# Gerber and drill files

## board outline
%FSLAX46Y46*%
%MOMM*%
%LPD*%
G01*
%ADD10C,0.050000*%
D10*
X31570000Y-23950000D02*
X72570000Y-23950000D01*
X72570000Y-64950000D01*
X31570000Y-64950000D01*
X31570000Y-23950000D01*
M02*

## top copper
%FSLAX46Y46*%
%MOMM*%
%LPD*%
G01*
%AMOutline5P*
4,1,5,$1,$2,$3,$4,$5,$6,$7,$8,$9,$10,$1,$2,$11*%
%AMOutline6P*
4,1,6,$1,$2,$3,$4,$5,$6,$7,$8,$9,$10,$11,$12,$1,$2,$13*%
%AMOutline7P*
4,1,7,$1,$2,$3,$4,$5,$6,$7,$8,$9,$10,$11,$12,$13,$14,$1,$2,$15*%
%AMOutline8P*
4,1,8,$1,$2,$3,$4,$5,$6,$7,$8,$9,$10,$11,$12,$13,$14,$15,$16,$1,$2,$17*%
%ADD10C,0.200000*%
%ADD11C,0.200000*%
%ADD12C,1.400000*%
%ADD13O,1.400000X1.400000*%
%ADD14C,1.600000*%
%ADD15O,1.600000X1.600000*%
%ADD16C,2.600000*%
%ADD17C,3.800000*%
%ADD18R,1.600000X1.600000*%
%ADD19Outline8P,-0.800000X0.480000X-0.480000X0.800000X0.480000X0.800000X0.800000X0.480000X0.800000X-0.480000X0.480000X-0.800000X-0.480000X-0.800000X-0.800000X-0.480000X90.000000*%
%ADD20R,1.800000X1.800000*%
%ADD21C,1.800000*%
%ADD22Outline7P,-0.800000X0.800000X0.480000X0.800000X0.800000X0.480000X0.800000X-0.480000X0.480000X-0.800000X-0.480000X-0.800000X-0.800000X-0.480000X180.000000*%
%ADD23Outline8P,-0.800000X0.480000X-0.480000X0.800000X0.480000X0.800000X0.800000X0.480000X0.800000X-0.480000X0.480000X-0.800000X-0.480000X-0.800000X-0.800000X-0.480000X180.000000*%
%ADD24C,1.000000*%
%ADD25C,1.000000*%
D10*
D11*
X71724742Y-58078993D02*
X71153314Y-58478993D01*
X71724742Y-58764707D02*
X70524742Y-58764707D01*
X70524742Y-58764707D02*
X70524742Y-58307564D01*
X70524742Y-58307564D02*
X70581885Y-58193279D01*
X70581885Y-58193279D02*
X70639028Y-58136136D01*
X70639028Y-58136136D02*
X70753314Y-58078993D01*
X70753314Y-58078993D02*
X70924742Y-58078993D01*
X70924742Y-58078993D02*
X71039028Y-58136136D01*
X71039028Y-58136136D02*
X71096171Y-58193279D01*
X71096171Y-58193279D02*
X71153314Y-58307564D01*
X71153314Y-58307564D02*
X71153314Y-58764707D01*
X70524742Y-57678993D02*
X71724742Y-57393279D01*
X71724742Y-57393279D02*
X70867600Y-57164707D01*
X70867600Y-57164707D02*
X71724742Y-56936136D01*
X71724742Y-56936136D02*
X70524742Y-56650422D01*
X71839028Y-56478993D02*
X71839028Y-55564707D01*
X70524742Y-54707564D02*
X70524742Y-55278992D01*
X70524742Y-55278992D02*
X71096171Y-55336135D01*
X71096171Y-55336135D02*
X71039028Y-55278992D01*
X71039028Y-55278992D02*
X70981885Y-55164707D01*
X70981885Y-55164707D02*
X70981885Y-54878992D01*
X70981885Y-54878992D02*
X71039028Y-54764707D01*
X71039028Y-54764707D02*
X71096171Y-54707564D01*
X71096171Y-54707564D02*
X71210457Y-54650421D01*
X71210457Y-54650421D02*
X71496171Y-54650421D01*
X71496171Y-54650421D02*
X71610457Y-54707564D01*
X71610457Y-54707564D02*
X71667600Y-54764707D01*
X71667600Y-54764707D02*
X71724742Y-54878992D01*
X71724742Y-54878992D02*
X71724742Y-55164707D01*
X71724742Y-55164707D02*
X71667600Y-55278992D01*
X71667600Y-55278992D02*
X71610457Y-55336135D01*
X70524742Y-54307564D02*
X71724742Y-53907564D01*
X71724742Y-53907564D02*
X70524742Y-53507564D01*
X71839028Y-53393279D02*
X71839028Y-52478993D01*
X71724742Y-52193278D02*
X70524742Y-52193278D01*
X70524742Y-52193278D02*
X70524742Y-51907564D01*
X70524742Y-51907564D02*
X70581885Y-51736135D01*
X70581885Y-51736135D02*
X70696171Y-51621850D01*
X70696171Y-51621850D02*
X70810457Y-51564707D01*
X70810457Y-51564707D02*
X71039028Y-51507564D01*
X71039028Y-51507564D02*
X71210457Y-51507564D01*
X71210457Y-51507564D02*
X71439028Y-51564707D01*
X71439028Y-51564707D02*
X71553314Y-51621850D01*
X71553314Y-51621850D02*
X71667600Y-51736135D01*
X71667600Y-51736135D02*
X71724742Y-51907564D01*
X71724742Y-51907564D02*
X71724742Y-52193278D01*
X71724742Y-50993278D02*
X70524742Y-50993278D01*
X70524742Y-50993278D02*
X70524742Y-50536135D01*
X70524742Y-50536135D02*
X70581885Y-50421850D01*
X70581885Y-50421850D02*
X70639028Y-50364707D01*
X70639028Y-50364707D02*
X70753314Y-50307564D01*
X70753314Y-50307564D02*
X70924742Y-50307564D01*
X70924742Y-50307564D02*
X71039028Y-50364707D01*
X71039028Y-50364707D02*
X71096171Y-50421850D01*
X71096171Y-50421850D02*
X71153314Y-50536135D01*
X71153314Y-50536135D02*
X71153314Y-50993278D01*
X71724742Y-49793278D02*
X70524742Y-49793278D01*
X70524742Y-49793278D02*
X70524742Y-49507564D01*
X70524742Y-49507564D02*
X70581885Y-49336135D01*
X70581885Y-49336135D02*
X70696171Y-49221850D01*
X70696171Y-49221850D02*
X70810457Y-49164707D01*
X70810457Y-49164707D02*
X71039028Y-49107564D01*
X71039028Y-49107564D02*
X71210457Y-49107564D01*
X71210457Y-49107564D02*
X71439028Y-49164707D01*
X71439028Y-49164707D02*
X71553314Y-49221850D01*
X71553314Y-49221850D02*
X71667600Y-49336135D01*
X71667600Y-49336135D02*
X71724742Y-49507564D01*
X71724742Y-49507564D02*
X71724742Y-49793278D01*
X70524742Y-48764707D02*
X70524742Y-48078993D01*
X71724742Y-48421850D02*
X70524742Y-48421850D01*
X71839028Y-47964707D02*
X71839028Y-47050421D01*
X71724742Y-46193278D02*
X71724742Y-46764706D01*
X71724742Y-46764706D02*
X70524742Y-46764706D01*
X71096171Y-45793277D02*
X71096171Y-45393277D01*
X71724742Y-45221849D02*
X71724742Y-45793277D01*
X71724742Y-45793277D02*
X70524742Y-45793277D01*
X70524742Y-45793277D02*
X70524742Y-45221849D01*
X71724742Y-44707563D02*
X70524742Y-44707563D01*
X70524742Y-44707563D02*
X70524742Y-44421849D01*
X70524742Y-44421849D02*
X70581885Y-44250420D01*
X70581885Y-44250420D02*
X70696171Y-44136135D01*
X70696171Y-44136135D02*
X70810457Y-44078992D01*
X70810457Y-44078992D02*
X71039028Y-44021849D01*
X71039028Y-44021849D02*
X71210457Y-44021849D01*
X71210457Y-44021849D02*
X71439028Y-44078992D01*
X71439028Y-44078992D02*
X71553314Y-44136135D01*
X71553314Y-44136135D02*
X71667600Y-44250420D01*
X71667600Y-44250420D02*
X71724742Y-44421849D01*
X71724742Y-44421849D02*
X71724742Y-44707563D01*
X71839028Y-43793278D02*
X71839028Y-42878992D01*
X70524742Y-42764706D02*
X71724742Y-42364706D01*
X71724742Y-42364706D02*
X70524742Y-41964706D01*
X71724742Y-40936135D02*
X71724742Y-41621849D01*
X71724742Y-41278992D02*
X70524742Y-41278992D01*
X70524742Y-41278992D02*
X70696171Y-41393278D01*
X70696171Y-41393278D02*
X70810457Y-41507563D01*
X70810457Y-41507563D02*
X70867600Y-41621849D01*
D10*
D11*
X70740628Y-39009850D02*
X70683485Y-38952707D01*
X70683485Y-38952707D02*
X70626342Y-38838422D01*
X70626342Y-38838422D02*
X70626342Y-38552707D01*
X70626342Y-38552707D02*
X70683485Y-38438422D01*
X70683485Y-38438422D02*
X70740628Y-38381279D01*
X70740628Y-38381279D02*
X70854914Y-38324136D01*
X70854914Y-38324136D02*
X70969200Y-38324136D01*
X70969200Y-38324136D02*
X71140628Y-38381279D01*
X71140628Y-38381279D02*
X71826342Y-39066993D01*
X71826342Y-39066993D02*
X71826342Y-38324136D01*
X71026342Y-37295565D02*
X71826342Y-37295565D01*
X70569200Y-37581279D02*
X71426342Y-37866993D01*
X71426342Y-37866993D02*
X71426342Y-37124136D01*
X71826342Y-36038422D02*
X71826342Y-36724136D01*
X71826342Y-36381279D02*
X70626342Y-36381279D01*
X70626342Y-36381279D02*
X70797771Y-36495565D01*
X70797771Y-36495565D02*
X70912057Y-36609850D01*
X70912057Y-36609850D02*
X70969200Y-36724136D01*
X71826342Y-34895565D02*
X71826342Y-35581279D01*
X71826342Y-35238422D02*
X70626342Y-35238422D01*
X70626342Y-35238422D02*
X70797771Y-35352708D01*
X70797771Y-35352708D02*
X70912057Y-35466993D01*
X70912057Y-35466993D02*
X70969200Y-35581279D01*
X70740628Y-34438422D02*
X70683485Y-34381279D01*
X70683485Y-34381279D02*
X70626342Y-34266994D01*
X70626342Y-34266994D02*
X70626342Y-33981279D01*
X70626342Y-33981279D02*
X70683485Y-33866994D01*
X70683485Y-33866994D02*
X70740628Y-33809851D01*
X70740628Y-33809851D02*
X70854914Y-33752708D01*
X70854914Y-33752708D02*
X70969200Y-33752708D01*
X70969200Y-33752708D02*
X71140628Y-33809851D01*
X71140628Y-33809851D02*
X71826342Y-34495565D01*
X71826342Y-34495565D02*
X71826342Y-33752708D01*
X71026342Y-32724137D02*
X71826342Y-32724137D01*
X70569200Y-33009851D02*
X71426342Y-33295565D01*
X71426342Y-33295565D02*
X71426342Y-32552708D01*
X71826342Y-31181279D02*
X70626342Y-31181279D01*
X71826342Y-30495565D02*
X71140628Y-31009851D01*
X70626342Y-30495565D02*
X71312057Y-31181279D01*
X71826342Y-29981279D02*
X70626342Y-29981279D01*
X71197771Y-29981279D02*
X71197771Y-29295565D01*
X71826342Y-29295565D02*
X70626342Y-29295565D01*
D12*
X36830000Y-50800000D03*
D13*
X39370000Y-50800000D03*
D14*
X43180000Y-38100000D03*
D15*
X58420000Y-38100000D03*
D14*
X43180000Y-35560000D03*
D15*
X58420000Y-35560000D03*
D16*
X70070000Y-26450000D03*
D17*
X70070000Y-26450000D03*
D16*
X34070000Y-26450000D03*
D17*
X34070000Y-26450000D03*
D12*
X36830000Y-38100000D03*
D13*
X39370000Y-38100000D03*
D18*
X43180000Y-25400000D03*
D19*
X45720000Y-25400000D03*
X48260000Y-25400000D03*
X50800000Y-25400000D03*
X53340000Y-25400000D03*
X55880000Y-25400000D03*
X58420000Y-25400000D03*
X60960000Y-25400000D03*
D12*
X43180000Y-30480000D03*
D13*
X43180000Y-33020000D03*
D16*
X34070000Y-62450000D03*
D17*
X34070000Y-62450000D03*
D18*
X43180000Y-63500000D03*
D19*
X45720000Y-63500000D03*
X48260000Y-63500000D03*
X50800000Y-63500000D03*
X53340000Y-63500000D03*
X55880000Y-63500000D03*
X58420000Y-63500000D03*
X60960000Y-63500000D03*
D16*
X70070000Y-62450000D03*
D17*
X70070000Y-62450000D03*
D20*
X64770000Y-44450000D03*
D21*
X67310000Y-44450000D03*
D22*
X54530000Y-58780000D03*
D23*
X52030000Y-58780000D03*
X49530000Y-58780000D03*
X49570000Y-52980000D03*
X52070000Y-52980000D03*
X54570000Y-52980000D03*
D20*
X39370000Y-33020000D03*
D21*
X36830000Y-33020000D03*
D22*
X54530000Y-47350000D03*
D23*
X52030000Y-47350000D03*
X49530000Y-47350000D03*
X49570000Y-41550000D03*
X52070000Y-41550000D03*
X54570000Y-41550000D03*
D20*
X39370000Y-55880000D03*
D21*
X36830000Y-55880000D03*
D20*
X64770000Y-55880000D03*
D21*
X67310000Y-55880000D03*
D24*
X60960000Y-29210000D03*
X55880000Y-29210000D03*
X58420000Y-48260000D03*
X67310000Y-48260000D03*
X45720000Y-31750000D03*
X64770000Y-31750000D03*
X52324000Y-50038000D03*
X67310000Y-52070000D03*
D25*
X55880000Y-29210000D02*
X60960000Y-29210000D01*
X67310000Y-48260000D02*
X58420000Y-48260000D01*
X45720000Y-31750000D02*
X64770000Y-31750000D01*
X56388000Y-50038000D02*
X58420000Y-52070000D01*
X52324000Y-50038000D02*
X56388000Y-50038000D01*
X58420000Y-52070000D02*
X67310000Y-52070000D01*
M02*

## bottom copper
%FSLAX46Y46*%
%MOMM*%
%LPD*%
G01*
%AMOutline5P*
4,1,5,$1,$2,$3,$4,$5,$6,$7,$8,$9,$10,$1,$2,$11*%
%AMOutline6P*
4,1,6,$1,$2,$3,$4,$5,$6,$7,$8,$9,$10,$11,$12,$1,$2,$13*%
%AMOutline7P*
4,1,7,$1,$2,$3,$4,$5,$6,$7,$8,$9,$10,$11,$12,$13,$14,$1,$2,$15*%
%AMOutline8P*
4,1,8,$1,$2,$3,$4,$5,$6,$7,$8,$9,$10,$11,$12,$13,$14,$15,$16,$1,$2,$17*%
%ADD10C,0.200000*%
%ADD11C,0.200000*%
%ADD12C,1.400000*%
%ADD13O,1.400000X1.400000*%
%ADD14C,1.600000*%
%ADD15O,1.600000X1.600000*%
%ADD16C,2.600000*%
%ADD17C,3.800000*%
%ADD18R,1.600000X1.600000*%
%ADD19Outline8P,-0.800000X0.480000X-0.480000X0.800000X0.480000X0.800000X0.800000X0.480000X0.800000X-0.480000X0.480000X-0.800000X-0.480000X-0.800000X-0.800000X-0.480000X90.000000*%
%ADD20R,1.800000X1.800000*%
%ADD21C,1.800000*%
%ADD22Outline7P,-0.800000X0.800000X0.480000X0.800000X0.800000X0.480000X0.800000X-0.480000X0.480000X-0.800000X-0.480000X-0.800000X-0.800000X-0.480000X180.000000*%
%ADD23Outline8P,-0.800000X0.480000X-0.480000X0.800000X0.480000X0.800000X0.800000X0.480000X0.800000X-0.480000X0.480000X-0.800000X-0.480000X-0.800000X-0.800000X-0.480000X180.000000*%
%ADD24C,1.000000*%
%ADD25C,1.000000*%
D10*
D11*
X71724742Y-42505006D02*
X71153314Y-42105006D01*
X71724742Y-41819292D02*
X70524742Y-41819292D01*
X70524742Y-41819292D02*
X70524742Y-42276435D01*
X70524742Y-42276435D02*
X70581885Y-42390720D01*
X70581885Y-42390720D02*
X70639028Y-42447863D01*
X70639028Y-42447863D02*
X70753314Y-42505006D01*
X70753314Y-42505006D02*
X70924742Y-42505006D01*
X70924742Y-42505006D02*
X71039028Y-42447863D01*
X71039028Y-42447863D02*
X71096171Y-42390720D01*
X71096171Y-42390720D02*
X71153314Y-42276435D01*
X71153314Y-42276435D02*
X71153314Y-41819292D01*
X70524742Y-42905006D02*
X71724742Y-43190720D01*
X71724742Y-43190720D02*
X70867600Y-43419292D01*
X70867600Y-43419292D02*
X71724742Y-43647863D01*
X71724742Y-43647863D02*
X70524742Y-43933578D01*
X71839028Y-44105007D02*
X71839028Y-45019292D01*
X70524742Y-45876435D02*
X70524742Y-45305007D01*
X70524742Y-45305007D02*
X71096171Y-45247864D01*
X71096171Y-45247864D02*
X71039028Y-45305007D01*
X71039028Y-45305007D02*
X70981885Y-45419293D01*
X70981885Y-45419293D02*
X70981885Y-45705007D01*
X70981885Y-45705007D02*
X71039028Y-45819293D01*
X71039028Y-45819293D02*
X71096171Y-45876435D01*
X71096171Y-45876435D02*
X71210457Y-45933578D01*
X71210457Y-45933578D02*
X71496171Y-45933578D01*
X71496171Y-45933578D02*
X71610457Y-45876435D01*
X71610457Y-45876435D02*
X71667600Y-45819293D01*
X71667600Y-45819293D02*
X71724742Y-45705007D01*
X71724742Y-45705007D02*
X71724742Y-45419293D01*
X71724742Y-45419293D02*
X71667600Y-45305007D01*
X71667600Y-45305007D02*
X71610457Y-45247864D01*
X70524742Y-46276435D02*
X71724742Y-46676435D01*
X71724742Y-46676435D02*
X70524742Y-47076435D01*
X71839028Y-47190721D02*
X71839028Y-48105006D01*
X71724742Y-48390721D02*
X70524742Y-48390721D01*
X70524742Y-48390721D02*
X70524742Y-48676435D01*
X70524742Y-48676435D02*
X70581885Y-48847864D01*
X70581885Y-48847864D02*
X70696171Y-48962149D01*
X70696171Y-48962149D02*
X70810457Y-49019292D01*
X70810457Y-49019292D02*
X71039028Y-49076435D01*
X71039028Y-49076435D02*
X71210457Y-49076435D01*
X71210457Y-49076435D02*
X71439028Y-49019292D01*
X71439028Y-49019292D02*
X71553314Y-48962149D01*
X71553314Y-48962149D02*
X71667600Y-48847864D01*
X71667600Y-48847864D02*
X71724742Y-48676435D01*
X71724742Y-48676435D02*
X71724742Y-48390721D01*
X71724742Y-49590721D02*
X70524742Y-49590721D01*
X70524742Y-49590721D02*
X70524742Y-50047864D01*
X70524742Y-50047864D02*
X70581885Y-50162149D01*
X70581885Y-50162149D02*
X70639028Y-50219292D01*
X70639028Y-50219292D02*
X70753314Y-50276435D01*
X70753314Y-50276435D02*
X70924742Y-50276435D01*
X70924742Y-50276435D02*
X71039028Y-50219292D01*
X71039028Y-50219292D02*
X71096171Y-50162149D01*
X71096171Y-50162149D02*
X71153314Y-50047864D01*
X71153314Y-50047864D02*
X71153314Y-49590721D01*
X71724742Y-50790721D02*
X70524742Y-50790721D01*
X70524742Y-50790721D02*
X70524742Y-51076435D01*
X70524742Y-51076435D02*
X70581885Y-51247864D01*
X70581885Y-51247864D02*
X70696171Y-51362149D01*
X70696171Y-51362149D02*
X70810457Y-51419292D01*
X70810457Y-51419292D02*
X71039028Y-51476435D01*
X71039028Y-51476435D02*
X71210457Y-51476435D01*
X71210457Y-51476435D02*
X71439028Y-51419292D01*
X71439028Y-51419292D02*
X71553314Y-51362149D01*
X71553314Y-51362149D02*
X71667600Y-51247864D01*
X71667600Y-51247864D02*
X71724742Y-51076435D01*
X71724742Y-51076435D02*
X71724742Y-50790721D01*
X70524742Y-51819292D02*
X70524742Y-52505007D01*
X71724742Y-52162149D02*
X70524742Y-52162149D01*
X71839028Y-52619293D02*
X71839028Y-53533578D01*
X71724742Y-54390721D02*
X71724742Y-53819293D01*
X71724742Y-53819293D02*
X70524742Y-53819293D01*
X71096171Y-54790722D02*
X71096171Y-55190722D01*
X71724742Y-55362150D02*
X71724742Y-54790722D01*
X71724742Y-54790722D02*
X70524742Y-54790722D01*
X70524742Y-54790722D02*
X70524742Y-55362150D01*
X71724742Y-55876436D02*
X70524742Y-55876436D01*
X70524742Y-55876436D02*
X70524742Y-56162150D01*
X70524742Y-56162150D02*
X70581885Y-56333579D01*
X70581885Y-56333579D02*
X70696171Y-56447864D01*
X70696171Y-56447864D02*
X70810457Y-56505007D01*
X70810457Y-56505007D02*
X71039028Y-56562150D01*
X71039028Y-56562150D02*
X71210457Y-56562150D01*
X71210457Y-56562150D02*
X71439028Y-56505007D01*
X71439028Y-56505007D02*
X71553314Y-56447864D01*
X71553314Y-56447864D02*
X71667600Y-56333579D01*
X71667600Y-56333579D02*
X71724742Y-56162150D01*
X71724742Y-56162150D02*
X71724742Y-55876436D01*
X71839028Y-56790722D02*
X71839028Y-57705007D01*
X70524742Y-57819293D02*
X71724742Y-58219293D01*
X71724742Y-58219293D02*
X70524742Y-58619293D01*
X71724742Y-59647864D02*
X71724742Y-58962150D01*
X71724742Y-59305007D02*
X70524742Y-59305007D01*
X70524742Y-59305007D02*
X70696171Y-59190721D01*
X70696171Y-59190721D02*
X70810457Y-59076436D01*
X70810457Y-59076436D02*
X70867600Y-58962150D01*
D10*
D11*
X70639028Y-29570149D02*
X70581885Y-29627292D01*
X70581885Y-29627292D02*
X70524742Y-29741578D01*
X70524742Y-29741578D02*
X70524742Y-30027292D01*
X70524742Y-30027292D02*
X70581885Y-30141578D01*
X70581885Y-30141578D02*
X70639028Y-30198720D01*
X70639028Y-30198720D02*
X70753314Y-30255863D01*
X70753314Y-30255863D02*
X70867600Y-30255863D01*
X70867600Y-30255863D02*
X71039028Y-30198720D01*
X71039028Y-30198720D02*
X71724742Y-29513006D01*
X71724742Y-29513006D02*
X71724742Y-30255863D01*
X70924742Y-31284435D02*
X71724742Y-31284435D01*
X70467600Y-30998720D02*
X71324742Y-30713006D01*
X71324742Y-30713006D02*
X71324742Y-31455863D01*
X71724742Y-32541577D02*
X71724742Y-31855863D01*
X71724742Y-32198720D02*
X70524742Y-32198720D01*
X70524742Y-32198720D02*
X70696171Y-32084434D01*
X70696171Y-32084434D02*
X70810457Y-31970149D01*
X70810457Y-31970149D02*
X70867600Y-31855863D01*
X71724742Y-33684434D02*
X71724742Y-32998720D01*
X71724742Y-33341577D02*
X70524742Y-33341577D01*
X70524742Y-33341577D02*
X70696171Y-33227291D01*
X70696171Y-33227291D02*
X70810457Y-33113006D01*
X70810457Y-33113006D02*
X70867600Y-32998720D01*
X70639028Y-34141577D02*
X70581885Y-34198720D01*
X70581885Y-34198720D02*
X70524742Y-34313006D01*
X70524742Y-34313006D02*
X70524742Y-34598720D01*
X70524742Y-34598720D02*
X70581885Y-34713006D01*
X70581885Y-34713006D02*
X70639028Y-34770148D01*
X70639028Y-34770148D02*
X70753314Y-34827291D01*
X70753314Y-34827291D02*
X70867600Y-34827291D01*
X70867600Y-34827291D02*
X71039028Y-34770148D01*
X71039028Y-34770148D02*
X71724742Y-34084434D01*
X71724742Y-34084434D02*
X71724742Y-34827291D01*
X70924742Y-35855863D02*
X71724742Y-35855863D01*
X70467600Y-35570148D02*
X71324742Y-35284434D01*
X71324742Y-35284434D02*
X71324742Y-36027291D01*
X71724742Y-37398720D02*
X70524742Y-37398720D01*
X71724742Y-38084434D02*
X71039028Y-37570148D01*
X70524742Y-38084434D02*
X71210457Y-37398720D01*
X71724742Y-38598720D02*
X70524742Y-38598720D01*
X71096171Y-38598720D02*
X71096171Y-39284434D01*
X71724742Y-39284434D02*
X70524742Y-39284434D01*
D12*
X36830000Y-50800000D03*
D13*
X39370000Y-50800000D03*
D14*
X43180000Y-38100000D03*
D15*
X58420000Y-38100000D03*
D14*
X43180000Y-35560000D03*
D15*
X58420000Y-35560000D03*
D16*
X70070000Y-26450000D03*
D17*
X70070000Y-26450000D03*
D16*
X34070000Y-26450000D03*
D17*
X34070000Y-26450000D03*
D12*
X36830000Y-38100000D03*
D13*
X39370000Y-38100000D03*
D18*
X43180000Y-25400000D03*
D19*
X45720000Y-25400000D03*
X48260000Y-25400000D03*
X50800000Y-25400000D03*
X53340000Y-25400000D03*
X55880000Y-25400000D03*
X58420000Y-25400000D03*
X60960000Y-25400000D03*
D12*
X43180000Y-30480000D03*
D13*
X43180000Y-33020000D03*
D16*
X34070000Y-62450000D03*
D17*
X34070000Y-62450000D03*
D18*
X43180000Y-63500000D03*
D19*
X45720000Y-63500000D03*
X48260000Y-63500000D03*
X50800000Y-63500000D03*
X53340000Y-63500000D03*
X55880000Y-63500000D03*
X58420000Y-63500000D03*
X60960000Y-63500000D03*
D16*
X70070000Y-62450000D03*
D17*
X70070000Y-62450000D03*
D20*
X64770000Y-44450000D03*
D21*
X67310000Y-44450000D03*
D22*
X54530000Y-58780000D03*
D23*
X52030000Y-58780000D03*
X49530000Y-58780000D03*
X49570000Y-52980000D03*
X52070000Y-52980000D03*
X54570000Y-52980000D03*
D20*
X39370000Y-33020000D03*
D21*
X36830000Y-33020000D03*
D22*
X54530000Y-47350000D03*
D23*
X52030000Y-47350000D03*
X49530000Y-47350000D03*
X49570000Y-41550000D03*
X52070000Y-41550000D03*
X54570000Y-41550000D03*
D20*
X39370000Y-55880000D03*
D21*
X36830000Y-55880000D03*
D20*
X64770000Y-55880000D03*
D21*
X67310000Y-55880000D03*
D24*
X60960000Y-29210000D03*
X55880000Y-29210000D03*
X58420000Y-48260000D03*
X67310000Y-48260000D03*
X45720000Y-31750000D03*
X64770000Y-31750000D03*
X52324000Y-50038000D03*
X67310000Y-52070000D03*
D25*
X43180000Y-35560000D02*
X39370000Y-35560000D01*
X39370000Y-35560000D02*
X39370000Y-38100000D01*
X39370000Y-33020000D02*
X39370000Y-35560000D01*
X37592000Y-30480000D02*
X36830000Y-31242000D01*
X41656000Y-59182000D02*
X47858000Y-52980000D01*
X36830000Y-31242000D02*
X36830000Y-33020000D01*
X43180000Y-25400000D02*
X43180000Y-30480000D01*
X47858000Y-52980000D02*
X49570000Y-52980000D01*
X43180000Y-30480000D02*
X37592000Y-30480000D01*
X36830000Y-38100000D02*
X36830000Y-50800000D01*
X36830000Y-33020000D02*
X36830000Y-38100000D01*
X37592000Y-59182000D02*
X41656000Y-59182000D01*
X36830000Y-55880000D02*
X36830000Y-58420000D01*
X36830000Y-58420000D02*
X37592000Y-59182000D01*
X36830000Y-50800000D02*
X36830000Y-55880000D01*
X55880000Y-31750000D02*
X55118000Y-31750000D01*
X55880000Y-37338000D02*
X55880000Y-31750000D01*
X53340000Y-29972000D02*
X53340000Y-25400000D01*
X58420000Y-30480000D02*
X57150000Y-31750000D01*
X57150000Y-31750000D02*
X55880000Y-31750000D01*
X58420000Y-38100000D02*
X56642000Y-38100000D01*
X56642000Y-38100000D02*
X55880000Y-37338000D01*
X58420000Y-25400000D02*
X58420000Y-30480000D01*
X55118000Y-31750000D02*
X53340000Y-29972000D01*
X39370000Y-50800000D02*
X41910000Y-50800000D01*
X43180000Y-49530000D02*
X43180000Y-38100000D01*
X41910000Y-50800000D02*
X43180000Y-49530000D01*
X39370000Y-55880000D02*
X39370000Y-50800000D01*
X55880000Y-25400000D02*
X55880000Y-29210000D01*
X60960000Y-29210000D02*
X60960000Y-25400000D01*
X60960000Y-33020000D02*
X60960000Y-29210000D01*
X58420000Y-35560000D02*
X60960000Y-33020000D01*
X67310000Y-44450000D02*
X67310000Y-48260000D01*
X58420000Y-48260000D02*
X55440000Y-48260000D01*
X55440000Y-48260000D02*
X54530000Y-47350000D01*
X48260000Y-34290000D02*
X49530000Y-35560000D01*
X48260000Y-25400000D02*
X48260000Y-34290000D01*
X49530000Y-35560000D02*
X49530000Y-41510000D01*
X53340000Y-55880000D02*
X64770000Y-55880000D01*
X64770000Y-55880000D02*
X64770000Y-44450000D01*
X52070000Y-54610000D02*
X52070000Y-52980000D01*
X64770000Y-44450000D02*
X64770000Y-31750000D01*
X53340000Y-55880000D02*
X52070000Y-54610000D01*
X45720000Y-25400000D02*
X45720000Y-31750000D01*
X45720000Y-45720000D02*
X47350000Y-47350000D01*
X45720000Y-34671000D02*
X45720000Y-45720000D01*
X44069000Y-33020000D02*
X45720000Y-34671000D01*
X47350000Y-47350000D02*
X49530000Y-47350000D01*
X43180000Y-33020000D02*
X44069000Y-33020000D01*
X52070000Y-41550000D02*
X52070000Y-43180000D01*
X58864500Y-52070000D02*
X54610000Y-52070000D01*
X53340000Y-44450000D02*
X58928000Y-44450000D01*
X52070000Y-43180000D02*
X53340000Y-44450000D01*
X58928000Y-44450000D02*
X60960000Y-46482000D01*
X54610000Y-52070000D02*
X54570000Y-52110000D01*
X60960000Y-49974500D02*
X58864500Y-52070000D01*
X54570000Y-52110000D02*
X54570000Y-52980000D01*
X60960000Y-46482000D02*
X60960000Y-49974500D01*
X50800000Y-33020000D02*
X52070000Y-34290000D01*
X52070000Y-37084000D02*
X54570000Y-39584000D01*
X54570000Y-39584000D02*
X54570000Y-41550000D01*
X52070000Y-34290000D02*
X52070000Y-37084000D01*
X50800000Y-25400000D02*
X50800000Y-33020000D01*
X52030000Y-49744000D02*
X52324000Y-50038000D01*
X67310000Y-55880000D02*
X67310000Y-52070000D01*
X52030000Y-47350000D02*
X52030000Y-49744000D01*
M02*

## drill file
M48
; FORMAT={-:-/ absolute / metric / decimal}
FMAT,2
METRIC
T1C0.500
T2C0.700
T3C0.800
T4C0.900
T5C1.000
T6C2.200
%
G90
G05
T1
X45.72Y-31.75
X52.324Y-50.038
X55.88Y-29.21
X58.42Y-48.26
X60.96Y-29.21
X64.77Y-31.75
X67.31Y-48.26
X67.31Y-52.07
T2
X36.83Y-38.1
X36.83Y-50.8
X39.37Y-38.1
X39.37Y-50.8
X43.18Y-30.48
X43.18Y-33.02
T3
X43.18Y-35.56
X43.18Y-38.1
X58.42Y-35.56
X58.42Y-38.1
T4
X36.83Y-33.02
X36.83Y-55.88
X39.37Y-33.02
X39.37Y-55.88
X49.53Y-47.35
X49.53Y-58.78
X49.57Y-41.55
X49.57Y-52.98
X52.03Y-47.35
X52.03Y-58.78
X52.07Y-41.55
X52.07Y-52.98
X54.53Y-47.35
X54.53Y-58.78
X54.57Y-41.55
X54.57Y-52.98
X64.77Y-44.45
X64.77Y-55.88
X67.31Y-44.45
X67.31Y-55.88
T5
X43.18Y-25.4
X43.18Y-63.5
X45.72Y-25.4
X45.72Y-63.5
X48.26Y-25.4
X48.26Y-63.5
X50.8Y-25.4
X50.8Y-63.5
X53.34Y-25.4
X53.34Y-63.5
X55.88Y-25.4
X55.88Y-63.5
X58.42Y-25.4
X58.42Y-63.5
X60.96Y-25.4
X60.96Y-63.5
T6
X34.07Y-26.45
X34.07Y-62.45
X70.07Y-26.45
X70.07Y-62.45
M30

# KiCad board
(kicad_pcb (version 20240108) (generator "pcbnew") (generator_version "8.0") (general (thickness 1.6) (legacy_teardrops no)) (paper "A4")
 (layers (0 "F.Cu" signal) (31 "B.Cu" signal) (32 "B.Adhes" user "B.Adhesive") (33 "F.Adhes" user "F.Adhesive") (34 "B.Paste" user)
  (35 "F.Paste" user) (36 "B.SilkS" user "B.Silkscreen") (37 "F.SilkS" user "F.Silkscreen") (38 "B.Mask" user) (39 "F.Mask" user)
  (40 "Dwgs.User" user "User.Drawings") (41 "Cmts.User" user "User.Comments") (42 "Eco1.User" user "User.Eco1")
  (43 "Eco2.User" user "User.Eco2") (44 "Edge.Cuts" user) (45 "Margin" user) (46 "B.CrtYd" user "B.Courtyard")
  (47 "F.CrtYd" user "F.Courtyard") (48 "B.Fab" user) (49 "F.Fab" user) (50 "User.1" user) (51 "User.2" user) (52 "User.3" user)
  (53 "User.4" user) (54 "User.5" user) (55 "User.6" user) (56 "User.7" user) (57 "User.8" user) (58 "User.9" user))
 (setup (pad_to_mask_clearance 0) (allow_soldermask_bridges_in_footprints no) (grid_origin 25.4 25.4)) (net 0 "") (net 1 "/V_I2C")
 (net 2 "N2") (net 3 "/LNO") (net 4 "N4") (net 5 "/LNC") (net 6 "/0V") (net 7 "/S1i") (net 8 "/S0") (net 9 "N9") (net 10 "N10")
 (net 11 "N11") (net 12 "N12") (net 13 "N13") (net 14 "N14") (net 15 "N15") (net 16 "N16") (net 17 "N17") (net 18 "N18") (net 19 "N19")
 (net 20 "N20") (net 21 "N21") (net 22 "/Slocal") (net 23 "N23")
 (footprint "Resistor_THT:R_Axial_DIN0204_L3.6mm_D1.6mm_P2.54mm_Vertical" (layer "F.Cu") (at 36.83 50.8)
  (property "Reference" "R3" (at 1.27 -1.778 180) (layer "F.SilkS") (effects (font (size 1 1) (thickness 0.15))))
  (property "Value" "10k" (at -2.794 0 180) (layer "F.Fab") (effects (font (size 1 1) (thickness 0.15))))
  (pad "1" thru_hole circle (at 0 0) (size 1.4 1.4) (drill 0.7) (layers "*.Cu" "*.Mask") (remove_unused_layers no) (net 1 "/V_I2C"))
  (pad "2" thru_hole oval (at 2.54 0) (size 1.4 1.4) (drill 0.7) (layers "*.Cu" "*.Mask") (remove_unused_layers no) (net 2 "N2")))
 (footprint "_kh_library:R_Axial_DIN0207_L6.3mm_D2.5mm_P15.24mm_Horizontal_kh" (layer "F.Cu") (at 43.18 38.1)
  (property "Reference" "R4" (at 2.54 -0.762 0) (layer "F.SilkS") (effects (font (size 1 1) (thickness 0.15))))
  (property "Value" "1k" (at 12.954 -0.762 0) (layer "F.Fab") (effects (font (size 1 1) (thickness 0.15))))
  (pad "1" thru_hole circle (at 0 0) (size 1.6 1.6) (drill 0.8) (layers "*.Cu" "*.Mask") (remove_unused_layers no) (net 2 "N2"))
  (pad "2" thru_hole oval (at 15.24 0) (size 1.6 1.6) (drill 0.8) (layers "*.Cu" "*.Mask") (remove_unused_layers no) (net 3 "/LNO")))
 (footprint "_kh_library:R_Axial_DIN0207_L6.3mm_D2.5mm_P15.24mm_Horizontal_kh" (layer "F.Cu") (at 43.18 35.56)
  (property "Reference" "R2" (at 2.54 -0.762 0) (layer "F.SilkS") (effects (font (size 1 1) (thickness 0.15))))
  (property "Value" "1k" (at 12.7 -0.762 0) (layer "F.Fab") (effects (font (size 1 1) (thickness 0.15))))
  (pad "1" thru_hole circle (at 0 0) (size 1.6 1.6) (drill 0.8) (layers "*.Cu" "*.Mask") (remove_unused_layers no) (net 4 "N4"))
  (pad "2" thru_hole oval (at 15.24 0) (size 1.6 1.6) (drill 0.8) (layers "*.Cu" "*.Mask") (remove_unused_layers no) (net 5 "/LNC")))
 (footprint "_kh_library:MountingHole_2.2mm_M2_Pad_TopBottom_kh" (layer "F.Cu") (at 70.07 26.45)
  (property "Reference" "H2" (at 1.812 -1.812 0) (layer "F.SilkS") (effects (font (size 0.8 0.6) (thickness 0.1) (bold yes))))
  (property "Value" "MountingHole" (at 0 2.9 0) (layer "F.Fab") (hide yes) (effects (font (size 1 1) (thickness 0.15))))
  (pad "1" thru_hole circle (at 0 0) (size 2.6 2.6) (drill 2.2) (layers "*.Cu" "*.Mask") (remove_unused_layers no))
  (pad "1" connect circle (at 0 0) (size 3.8 3.8) (layers "F.Cu" "F.Mask"))
  (pad "1" connect circle (at 0 0) (size 3.8 3.8) (layers "B.Cu" "B.Mask")))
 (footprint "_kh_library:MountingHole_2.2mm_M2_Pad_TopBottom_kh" (layer "F.Cu") (at 34.07 26.45)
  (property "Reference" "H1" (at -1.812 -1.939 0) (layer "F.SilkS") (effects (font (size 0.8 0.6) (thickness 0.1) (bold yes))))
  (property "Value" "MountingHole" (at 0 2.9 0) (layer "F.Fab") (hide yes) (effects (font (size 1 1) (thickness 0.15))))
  (pad "1" thru_hole circle (at 0 0) (size 2.6 2.6) (drill 2.2) (layers "*.Cu" "*.Mask") (remove_unused_layers no))
  (pad "1" connect circle (at 0 0) (size 3.8 3.8) (layers "F.Cu" "F.Mask"))
  (pad "1" connect circle (at 0 0) (size 3.8 3.8) (layers "B.Cu" "B.Mask")))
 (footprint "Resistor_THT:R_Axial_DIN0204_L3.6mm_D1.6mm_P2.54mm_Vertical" (layer "F.Cu") (at 36.83 38.1)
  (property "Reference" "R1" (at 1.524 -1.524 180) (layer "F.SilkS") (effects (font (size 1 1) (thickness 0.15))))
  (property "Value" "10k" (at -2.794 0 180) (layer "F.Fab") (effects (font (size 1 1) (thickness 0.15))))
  (pad "1" thru_hole circle (at 0 0) (size 1.4 1.4) (drill 0.7) (layers "*.Cu" "*.Mask") (remove_unused_layers no) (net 1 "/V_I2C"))
  (pad "2" thru_hole oval (at 2.54 0) (size 1.4 1.4) (drill 0.7) (layers "*.Cu" "*.Mask") (remove_unused_layers no) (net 4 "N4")))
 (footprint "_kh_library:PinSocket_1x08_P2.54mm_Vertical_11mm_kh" (layer "F.Cu") (at 43.18 25.4 90)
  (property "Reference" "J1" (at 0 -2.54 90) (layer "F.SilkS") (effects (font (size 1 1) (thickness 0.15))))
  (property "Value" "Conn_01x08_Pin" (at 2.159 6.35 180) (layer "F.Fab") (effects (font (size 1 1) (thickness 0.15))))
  (pad "1" thru_hole rect (at 0 0 90) (size 1.6 1.6) (drill 1) (layers "*.Cu" "*.Mask") (remove_unused_layers no) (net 1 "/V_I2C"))
  (pad "2" thru_hole roundrect (at 0 2.54 90) (size 1.6 1.6) (drill 1) (layers "*.Cu" "*.Mask") (remove_unused_layers no)
   (roundrect_rratio 0) (chamfer_ratio 0.2) (chamfer top_left top_right bottom_left bottom_right) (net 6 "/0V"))
  (pad "3" thru_hole roundrect (at 0 5.08 90) (size 1.6 1.6) (drill 1) (layers "*.Cu" "*.Mask") (remove_unused_layers no)
   (roundrect_rratio 0) (chamfer_ratio 0.2) (chamfer top_left top_right bottom_left bottom_right) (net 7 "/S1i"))
  (pad "4" thru_hole roundrect (at 0 7.62 90) (size 1.6 1.6) (drill 1) (layers "*.Cu" "*.Mask") (remove_unused_layers no)
   (roundrect_rratio 0) (chamfer_ratio 0.2) (chamfer top_left top_right bottom_left bottom_right) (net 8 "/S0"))
  (pad "5" thru_hole roundrect (at 0 10.16 90) (size 1.6 1.6) (drill 1) (layers "*.Cu" "*.Mask") (remove_unused_layers no)
   (roundrect_rratio 0) (chamfer_ratio 0.2) (chamfer top_left top_right bottom_left bottom_right) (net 3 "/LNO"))
  (pad "6" thru_hole roundrect (at 0 12.7 90) (size 1.6 1.6) (drill 1) (layers "*.Cu" "*.Mask") (remove_unused_layers no)
   (roundrect_rratio 0) (chamfer_ratio 0.2) (chamfer top_left top_right bottom_left bottom_right) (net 5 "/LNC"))
  (pad "7" thru_hole roundrect (at 0 15.24 90) (size 1.6 1.6) (drill 1) (layers "*.Cu" "*.Mask") (remove_unused_layers no)
   (roundrect_rratio 0) (chamfer_ratio 0.2) (chamfer top_left top_right bottom_left bottom_right) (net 3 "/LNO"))
  (pad "8" thru_hole roundrect (at 0 17.78 90) (size 1.6 1.6) (drill 1) (layers "*.Cu" "*.Mask") (remove_unused_layers no)
   (roundrect_rratio 0) (chamfer_ratio 0.2) (chamfer top_left top_right bottom_left bottom_right) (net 5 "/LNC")))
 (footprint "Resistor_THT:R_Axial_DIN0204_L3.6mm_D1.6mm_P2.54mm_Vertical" (layer "F.Cu") (at 43.18 30.48 -90)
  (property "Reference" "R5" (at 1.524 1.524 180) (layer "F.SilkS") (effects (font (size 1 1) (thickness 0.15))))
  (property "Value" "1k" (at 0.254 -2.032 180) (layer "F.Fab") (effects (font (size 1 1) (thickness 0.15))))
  (pad "1" thru_hole circle (at 0 0 270) (size 1.4 1.4) (drill 0.7) (layers "*.Cu" "*.Mask") (remove_unused_layers no) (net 1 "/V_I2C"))
  (pad "2" thru_hole oval (at 2.54 0 270) (size 1.4 1.4) (drill 0.7) (layers "*.Cu" "*.Mask") (remove_unused_layers no) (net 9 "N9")))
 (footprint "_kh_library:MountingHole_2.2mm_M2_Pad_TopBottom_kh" (layer "F.Cu") (at 34.07 62.45)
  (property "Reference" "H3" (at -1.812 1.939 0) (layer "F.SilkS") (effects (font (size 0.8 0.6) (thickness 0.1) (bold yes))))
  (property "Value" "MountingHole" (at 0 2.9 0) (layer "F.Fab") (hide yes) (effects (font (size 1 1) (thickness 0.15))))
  (pad "1" thru_hole circle (at 0 0) (size 2.6 2.6) (drill 2.2) (layers "*.Cu" "*.Mask") (remove_unused_layers no))
  (pad "1" connect circle (at 0 0) (size 3.8 3.8) (layers "F.Cu" "F.Mask"))
  (pad "1" connect circle (at 0 0) (size 3.8 3.8) (layers "B.Cu" "B.Mask")))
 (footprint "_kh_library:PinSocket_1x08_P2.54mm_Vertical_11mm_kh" (layer "F.Cu") (at 43.18 63.5 90)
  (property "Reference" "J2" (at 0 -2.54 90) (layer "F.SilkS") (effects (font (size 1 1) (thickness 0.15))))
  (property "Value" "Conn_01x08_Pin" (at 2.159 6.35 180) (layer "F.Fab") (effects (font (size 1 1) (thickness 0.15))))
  (pad "1" thru_hole rect (at 0 0 90) (size 1.6 1.6) (drill 1) (layers "*.Cu" "*.Mask") (remove_unused_layers no) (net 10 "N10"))
  (pad "2" thru_hole roundrect (at 0 2.54 90) (size 1.6 1.6) (drill 1) (layers "*.Cu" "*.Mask") (remove_unused_layers no)
   (roundrect_rratio 0) (chamfer_ratio 0.2) (chamfer top_left top_right bottom_left bottom_right) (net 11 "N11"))
  (pad "3" thru_hole roundrect (at 0 5.08 90) (size 1.6 1.6) (drill 1) (layers "*.Cu" "*.Mask") (remove_unused_layers no)
   (roundrect_rratio 0) (chamfer_ratio 0.2) (chamfer top_left top_right bottom_left bottom_right) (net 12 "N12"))
  (pad "4" thru_hole roundrect (at 0 7.62 90) (size 1.6 1.6) (drill 1) (layers "*.Cu" "*.Mask") (remove_unused_layers no)
   (roundrect_rratio 0) (chamfer_ratio 0.2) (chamfer top_left top_right bottom_left bottom_right) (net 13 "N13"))
  (pad "5" thru_hole roundrect (at 0 10.16 90) (size 1.6 1.6) (drill 1) (layers "*.Cu" "*.Mask") (remove_unused_layers no)
   (roundrect_rratio 0) (chamfer_ratio 0.2) (chamfer top_left top_right bottom_left bottom_right) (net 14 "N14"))
  (pad "6" thru_hole roundrect (at 0 12.7 90) (size 1.6 1.6) (drill 1) (layers "*.Cu" "*.Mask") (remove_unused_layers no)
   (roundrect_rratio 0) (chamfer_ratio 0.2) (chamfer top_left top_right bottom_left bottom_right) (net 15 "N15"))
  (pad "7" thru_hole roundrect (at 0 15.24 90) (size 1.6 1.6) (drill 1) (layers "*.Cu" "*.Mask") (remove_unused_layers no)
   (roundrect_rratio 0) (chamfer_ratio 0.2) (chamfer top_left top_right bottom_left bottom_right) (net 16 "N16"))
  (pad "8" thru_hole roundrect (at 0 17.78 90) (size 1.6 1.6) (drill 1) (layers "*.Cu" "*.Mask") (remove_unused_layers no)
   (roundrect_rratio 0) (chamfer_ratio 0.2) (chamfer top_left top_right bottom_left bottom_right) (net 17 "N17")))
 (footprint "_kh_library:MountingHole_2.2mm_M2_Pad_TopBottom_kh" (layer "F.Cu") (at 70.07 62.45)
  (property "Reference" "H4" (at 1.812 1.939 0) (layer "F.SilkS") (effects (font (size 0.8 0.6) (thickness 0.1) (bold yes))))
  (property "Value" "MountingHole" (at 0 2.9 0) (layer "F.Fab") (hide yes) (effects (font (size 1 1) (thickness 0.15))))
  (pad "1" thru_hole circle (at 0 0) (size 2.6 2.6) (drill 2.2) (layers "*.Cu" "*.Mask") (remove_unused_layers no))
  (pad "1" connect circle (at 0 0) (size 3.8 3.8) (layers "F.Cu" "F.Mask"))
  (pad "1" connect circle (at 0 0) (size 3.8 3.8) (layers "B.Cu" "B.Mask")))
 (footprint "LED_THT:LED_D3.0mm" (layer "B.Cu") (at 64.77 44.45)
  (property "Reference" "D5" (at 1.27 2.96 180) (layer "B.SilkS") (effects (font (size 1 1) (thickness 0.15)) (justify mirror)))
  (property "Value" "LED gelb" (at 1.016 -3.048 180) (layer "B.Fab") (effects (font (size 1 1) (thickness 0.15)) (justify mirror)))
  (pad "1" thru_hole rect (at 0 0) (size 1.8 1.8) (drill 0.9) (layers "*.Cu" "*.Mask") (remove_unused_layers no) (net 6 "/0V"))
  (pad "2" thru_hole circle (at 2.54 0) (size 1.8 1.8) (drill 0.9) (layers "*.Cu" "*.Mask") (remove_unused_layers no) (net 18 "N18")))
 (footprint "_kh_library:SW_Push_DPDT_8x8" (layer "B.Cu") (at 54.57 58.78 180)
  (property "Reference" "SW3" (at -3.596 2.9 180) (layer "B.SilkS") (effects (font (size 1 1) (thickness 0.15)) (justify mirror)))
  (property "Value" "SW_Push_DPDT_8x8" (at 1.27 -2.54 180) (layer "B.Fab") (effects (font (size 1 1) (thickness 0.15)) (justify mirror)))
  (pad "1" thru_hole roundrect (at 0.04 0 180) (size 1.6 1.6) (drill 0.9) (layers "*.Cu" "*.Mask") (remove_unused_layers no)
   (roundrect_rratio 0) (chamfer_ratio 0.2) (chamfer top_right bottom_left bottom_right) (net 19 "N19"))
  (pad "2" thru_hole roundrect (at 2.54 0 180) (size 1.6 1.6) (drill 0.9) (layers "*.Cu" "*.Mask") (remove_unused_layers no)
   (roundrect_rratio 0) (chamfer_ratio 0.2) (chamfer top_left top_right bottom_left bottom_right) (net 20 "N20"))
  (pad "3" thru_hole roundrect (at 5.04 0 180) (size 1.6 1.6) (drill 0.9) (layers "*.Cu" "*.Mask") (remove_unused_layers no)
   (roundrect_rratio 0) (chamfer_ratio 0.2) (chamfer top_left top_right bottom_left bottom_right) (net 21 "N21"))
  (pad "4" thru_hole roundrect (at 5 5.8 180) (size 1.6 1.6) (drill 0.9) (layers "*.Cu" "*.Mask") (remove_unused_layers no)
   (roundrect_rratio 0) (chamfer_ratio 0.2) (chamfer top_left top_right bottom_left bottom_right) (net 1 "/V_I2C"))
  (pad "5" thru_hole roundrect (at 2.5 5.8 180) (size 1.6 1.6) (drill 0.9) (layers "*.Cu" "*.Mask") (remove_unused_layers no)
   (roundrect_rratio 0) (chamfer_ratio 0.2) (chamfer top_left top_right bottom_left bottom_right) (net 6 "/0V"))
  (pad "6" thru_hole roundrect (at 0 5.8 180) (size 1.6 1.6) (drill 0.9) (layers "*.Cu" "*.Mask") (remove_unused_layers no)
   (roundrect_rratio 0) (chamfer_ratio 0.2) (chamfer top_left top_right bottom_left bottom_right) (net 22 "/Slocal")))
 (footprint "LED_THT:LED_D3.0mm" (layer "B.Cu") (at 39.37 33.02 180)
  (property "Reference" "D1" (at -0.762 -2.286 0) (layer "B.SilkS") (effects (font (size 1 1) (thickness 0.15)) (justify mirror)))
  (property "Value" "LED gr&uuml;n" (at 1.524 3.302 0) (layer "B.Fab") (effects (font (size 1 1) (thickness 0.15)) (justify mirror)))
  (pad "1" thru_hole rect (at 0 0 180) (size 1.8 1.8) (drill 0.9) (layers "*.Cu" "*.Mask") (remove_unused_layers no) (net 4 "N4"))
  (pad "2" thru_hole circle (at 2.54 0 180) (size 1.8 1.8) (drill 0.9) (layers "*.Cu" "*.Mask") (remove_unused_layers no) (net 1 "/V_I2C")))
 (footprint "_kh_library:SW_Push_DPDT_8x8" (layer "B.Cu") (at 54.57 47.35 180)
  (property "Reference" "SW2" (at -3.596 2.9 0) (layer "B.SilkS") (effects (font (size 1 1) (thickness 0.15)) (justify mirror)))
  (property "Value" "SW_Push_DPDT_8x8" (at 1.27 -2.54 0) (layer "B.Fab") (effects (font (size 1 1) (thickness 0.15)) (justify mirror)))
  (pad "1" thru_hole roundrect (at 0.04 0 180) (size 1.6 1.6) (drill 0.9) (layers "*.Cu" "*.Mask") (remove_unused_layers no)
   (roundrect_rratio 0) (chamfer_ratio 0.2) (chamfer top_right bottom_left bottom_right) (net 18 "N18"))
  (pad "2" thru_hole roundrect (at 2.54 0 180) (size 1.6 1.6) (drill 0.9) (layers "*.Cu" "*.Mask") (remove_unused_layers no)
   (roundrect_rratio 0) (chamfer_ratio 0.2) (chamfer top_left top_right bottom_left bottom_right) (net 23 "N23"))
  (pad "3" thru_hole roundrect (at 5.04 0 180) (size 1.6 1.6) (drill 0.9) (layers "*.Cu" "*.Mask") (remove_unused_layers no)
   (roundrect_rratio 0) (chamfer_ratio 0.2) (chamfer top_left top_right bottom_left bottom_right) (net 9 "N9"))
  (pad "4" thru_hole roundrect (at 5 5.8 180) (size 1.6 1.6) (drill 0.9) (layers "*.Cu" "*.Mask") (remove_unused_layers no)
   (roundrect_rratio 0) (chamfer_ratio 0.2) (chamfer top_left top_right bottom_left bottom_right) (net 7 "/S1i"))
  (pad "5" thru_hole roundrect (at 2.5 5.8 180) (size 1.6 1.6) (drill 0.9) (layers "*.Cu" "*.Mask") (remove_unused_layers no)
   (roundrect_rratio 0) (chamfer_ratio 0.2) (chamfer top_left top_right bottom_left bottom_right) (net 22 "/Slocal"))
  (pad "6" thru_hole roundrect (at 0 5.8 180) (size 1.6 1.6) (drill 0.9) (layers "*.Cu" "*.Mask") (remove_unused_layers no)
   (roundrect_rratio 0) (chamfer_ratio 0.2) (chamfer top_left top_right bottom_left bottom_right) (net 8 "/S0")))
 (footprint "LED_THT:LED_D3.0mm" (layer "B.Cu") (at 39.37 55.88 180)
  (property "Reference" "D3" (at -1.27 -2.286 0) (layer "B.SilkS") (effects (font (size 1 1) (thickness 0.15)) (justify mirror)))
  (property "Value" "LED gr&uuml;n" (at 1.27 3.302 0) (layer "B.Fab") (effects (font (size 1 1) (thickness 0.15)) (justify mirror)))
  (pad "1" thru_hole rect (at 0 0 180) (size 1.8 1.8) (drill 0.9) (layers "*.Cu" "*.Mask") (remove_unused_layers no) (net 2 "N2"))
  (pad "2" thru_hole circle (at 2.54 0 180) (size 1.8 1.8) (drill 0.9) (layers "*.Cu" "*.Mask") (remove_unused_layers no) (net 1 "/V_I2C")))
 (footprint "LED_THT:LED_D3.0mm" (layer "B.Cu") (at 64.77 55.88)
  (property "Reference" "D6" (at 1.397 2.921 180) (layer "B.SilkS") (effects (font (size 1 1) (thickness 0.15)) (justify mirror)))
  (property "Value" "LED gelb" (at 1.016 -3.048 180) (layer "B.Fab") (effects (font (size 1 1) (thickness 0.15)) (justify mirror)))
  (pad "1" thru_hole rect (at 0 0) (size 1.8 1.8) (drill 0.9) (layers "*.Cu" "*.Mask") (remove_unused_layers no) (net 6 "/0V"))
  (pad "2" thru_hole circle (at 2.54 0) (size 1.8 1.8) (drill 0.9) (layers "*.Cu" "*.Mask") (remove_unused_layers no) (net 23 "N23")))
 (gr_rect (start 31.57 23.95) (end 72.57 64.95) (stroke (width 0.05) (type default)) (fill none) (layer "Edge.Cuts"))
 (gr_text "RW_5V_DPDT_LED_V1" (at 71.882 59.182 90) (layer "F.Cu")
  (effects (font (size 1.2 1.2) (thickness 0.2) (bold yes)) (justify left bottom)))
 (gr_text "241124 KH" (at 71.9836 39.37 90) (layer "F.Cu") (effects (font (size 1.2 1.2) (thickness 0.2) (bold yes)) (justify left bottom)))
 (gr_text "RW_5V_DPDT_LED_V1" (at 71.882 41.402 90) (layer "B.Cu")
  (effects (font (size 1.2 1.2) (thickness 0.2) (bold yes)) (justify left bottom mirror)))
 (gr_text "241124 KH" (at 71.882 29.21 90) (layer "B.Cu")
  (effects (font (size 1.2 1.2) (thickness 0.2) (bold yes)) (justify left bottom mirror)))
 (segment (start 43.18 35.56) (end 39.37 35.56) (width 1) (layer "B.Cu") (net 4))
 (segment (start 39.37 35.56) (end 39.37 38.1) (width 1) (layer "B.Cu") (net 4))
 (segment (start 39.37 33.02) (end 39.37 35.56) (width 1) (layer "B.Cu") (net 4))
 (segment (start 37.592 30.48) (end 36.83 31.242) (width 1) (layer "B.Cu") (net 1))
 (segment (start 41.656 59.182) (end 47.858 52.98) (width 1) (layer "B.Cu") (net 1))
 (segment (start 36.83 31.242) (end 36.83 33.02) (width 1) (layer "B.Cu") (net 1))
 (segment (start 43.18 25.4) (end 43.18 30.48) (width 1) (layer "B.Cu") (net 1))
 (segment (start 47.858 52.98) (end 49.57 52.98) (width 1) (layer "B.Cu") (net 1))
 (segment (start 43.18 30.48) (end 37.592 30.48) (width 1) (layer "B.Cu") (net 1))
 (segment (start 36.83 38.1) (end 36.83 50.8) (width 1) (layer "B.Cu") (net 1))
 (segment (start 36.83 33.02) (end 36.83 38.1) (width 1) (layer "B.Cu") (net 1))
 (segment (start 37.592 59.182) (end 41.656 59.182) (width 1) (layer "B.Cu") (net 1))
 (segment (start 36.83 55.88) (end 36.83 58.42) (width 1) (layer "B.Cu") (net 1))
 (segment (start 36.83 58.42) (end 37.592 59.182) (width 1) (layer "B.Cu") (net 1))
 (segment (start 36.83 50.8) (end 36.83 55.88) (width 1) (layer "B.Cu") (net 1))
 (segment (start 55.88 31.75) (end 55.118 31.75) (width 1) (layer "B.Cu") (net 3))
 (segment (start 55.88 37.338) (end 55.88 31.75) (width 1) (layer "B.Cu") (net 3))
 (segment (start 53.34 29.972) (end 53.34 25.4) (width 1) (layer "B.Cu") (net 3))
 (segment (start 58.42 30.48) (end 57.15 31.75) (width 1) (layer "B.Cu") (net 3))
 (segment (start 57.15 31.75) (end 55.88 31.75) (width 1) (layer "B.Cu") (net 3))
 (segment (start 58.42 38.1) (end 56.642 38.1) (width 1) (layer "B.Cu") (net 3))
 (segment (start 56.642 38.1) (end 55.88 37.338) (width 1) (layer "B.Cu") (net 3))
 (segment (start 58.42 25.4) (end 58.42 30.48) (width 1) (layer "B.Cu") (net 3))
 (segment (start 55.118 31.75) (end 53.34 29.972) (width 1) (layer "B.Cu") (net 3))
 (segment (start 39.37 50.8) (end 41.91 50.8) (width 1) (layer "B.Cu") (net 2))
 (segment (start 43.18 49.53) (end 43.18 38.1) (width 1) (layer "B.Cu") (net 2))
 (segment (start 41.91 50.8) (end 43.18 49.53) (width 1) (layer "B.Cu") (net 2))
 (segment (start 39.37 55.88) (end 39.37 50.8) (width 1) (layer "B.Cu") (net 2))
 (segment (start 55.88 29.21) (end 60.96 29.21) (width 1) (layer "F.Cu") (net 5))
 (via (at 60.96 29.21) (size 1) (drill 0.5) (layers "F.Cu" "B.Cu") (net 5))
 (via (at 55.88 29.21) (size 1) (drill 0.5) (layers "F.Cu" "B.Cu") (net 5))
 (segment (start 55.88 25.4) (end 55.88 29.21) (width 1) (layer "B.Cu") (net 5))
 (segment (start 60.96 29.21) (end 60.96 25.4) (width 1) (layer "B.Cu") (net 5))
 (segment (start 60.96 33.02) (end 60.96 29.21) (width 1) (layer "B.Cu") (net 5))
 (segment (start 58.42 35.56) (end 60.96 33.02) (width 1) (layer "B.Cu") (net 5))
 (segment (start 67.31 48.26) (end 58.42 48.26) (width 1) (layer "F.Cu") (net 18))
 (via (at 58.42 48.26) (size 1) (drill 0.5) (layers "F.Cu" "B.Cu") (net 18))
 (via (at 67.31 48.26) (size 1) (drill 0.5) (layers "F.Cu" "B.Cu") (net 18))
 (segment (start 67.31 44.45) (end 67.31 48.26) (width 1) (layer "B.Cu") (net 18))
 (segment (start 58.42 48.26) (end 55.44 48.26) (width 1) (layer "B.Cu") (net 18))
 (segment (start 55.44 48.26) (end 54.53 47.35) (width 1) (layer "B.Cu") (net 18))
 (segment (start 48.26 34.29) (end 49.53 35.56) (width 1) (layer "B.Cu") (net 7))
 (segment (start 48.26 25.4) (end 48.26 34.29) (width 1) (layer "B.Cu") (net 7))
 (segment (start 49.53 35.56) (end 49.53 41.51) (width 1) (layer "B.Cu") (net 7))
 (segment (start 45.72 31.75) (end 64.77 31.75) (width 1) (layer "F.Cu") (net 6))
 (via (at 45.72 31.75) (size 1) (drill 0.5) (layers "F.Cu" "B.Cu") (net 6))
 (via (at 64.77 31.75) (size 1) (drill 0.5) (layers "F.Cu" "B.Cu") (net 6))
 (segment (start 53.34 55.88) (end 64.77 55.88) (width 1) (layer "B.Cu") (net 6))
 (segment (start 64.77 55.88) (end 64.77 44.45) (width 1) (layer "B.Cu") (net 6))
 (segment (start 52.07 54.61) (end 52.07 52.98) (width 1) (layer "B.Cu") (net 6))
 (segment (start 64.77 44.45) (end 64.77 31.75) (width 1) (layer "B.Cu") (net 6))
 (segment (start 53.34 55.88) (end 52.07 54.61) (width 1) (layer "B.Cu") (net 6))
 (segment (start 45.72 25.4) (end 45.72 31.75) (width 1) (layer "B.Cu") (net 6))
 (segment (start 45.72 45.72) (end 47.35 47.35) (width 1) (layer "B.Cu") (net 9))
 (segment (start 45.72 34.671) (end 45.72 45.72) (width 1) (layer "B.Cu") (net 9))
 (segment (start 44.069 33.02) (end 45.72 34.671) (width 1) (layer "B.Cu") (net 9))
 (segment (start 47.35 47.35) (end 49.53 47.35) (width 1) (layer "B.Cu") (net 9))
 (segment (start 43.18 33.02) (end 44.069 33.02) (width 1) (layer "B.Cu") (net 9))
 (segment (start 52.07 41.55) (end 52.07 43.18) (width 1) (layer "B.Cu") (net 22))
 (segment (start 58.8645 52.07) (end 54.61 52.07) (width 1) (layer "B.Cu") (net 22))
 (segment (start 53.34 44.45) (end 58.928 44.45) (width 1) (layer "B.Cu") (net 22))
 (segment (start 52.07 43.18) (end 53.34 44.45) (width 1) (layer "B.Cu") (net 22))
 (segment (start 58.928 44.45) (end 60.96 46.482) (width 1) (layer "B.Cu") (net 22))
 (segment (start 54.61 52.07) (end 54.57 52.11) (width 1) (layer "B.Cu") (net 22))
 (segment (start 60.96 49.9745) (end 58.8645 52.07) (width 1) (layer "B.Cu") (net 22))
 (segment (start 54.57 52.11) (end 54.57 52.98) (width 1) (layer "B.Cu") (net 22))
 (segment (start 60.96 46.482) (end 60.96 49.9745) (width 1) (layer "B.Cu") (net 22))
 (segment (start 50.8 33.02) (end 52.07 34.29) (width 1) (layer "B.Cu") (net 8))
 (segment (start 52.07 37.084) (end 54.57 39.584) (width 1) (layer "B.Cu") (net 8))
 (segment (start 54.57 39.584) (end 54.57 41.55) (width 1) (layer "B.Cu") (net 8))
 (segment (start 52.07 34.29) (end 52.07 37.084) (width 1) (layer "B.Cu") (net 8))
 (segment (start 50.8 25.4) (end 50.8 33.02) (width 1) (layer "B.Cu") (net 8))
 (segment (start 56.388 50.038) (end 58.42 52.07) (width 1) (layer "F.Cu") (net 23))
 (segment (start 52.324 50.038) (end 56.388 50.038) (width 1) (layer "F.Cu") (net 23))
 (segment (start 58.42 52.07) (end 67.31 52.07) (width 1) (layer "F.Cu") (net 23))
 (via (at 52.324 50.038) (size 1) (drill 0.5) (layers "F.Cu" "B.Cu") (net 23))
 (via (at 67.31 52.07) (size 1) (drill 0.5) (layers "F.Cu" "B.Cu") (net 23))
 (segment (start 52.03 49.744) (end 52.324 50.038) (width 1) (layer "B.Cu") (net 23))
 (segment (start 67.31 55.88) (end 67.31 52.07) (width 1) (layer "B.Cu") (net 23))
 (segment (start 52.03 47.35) (end 52.03 49.744) (width 1) (layer "B.Cu") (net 23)))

